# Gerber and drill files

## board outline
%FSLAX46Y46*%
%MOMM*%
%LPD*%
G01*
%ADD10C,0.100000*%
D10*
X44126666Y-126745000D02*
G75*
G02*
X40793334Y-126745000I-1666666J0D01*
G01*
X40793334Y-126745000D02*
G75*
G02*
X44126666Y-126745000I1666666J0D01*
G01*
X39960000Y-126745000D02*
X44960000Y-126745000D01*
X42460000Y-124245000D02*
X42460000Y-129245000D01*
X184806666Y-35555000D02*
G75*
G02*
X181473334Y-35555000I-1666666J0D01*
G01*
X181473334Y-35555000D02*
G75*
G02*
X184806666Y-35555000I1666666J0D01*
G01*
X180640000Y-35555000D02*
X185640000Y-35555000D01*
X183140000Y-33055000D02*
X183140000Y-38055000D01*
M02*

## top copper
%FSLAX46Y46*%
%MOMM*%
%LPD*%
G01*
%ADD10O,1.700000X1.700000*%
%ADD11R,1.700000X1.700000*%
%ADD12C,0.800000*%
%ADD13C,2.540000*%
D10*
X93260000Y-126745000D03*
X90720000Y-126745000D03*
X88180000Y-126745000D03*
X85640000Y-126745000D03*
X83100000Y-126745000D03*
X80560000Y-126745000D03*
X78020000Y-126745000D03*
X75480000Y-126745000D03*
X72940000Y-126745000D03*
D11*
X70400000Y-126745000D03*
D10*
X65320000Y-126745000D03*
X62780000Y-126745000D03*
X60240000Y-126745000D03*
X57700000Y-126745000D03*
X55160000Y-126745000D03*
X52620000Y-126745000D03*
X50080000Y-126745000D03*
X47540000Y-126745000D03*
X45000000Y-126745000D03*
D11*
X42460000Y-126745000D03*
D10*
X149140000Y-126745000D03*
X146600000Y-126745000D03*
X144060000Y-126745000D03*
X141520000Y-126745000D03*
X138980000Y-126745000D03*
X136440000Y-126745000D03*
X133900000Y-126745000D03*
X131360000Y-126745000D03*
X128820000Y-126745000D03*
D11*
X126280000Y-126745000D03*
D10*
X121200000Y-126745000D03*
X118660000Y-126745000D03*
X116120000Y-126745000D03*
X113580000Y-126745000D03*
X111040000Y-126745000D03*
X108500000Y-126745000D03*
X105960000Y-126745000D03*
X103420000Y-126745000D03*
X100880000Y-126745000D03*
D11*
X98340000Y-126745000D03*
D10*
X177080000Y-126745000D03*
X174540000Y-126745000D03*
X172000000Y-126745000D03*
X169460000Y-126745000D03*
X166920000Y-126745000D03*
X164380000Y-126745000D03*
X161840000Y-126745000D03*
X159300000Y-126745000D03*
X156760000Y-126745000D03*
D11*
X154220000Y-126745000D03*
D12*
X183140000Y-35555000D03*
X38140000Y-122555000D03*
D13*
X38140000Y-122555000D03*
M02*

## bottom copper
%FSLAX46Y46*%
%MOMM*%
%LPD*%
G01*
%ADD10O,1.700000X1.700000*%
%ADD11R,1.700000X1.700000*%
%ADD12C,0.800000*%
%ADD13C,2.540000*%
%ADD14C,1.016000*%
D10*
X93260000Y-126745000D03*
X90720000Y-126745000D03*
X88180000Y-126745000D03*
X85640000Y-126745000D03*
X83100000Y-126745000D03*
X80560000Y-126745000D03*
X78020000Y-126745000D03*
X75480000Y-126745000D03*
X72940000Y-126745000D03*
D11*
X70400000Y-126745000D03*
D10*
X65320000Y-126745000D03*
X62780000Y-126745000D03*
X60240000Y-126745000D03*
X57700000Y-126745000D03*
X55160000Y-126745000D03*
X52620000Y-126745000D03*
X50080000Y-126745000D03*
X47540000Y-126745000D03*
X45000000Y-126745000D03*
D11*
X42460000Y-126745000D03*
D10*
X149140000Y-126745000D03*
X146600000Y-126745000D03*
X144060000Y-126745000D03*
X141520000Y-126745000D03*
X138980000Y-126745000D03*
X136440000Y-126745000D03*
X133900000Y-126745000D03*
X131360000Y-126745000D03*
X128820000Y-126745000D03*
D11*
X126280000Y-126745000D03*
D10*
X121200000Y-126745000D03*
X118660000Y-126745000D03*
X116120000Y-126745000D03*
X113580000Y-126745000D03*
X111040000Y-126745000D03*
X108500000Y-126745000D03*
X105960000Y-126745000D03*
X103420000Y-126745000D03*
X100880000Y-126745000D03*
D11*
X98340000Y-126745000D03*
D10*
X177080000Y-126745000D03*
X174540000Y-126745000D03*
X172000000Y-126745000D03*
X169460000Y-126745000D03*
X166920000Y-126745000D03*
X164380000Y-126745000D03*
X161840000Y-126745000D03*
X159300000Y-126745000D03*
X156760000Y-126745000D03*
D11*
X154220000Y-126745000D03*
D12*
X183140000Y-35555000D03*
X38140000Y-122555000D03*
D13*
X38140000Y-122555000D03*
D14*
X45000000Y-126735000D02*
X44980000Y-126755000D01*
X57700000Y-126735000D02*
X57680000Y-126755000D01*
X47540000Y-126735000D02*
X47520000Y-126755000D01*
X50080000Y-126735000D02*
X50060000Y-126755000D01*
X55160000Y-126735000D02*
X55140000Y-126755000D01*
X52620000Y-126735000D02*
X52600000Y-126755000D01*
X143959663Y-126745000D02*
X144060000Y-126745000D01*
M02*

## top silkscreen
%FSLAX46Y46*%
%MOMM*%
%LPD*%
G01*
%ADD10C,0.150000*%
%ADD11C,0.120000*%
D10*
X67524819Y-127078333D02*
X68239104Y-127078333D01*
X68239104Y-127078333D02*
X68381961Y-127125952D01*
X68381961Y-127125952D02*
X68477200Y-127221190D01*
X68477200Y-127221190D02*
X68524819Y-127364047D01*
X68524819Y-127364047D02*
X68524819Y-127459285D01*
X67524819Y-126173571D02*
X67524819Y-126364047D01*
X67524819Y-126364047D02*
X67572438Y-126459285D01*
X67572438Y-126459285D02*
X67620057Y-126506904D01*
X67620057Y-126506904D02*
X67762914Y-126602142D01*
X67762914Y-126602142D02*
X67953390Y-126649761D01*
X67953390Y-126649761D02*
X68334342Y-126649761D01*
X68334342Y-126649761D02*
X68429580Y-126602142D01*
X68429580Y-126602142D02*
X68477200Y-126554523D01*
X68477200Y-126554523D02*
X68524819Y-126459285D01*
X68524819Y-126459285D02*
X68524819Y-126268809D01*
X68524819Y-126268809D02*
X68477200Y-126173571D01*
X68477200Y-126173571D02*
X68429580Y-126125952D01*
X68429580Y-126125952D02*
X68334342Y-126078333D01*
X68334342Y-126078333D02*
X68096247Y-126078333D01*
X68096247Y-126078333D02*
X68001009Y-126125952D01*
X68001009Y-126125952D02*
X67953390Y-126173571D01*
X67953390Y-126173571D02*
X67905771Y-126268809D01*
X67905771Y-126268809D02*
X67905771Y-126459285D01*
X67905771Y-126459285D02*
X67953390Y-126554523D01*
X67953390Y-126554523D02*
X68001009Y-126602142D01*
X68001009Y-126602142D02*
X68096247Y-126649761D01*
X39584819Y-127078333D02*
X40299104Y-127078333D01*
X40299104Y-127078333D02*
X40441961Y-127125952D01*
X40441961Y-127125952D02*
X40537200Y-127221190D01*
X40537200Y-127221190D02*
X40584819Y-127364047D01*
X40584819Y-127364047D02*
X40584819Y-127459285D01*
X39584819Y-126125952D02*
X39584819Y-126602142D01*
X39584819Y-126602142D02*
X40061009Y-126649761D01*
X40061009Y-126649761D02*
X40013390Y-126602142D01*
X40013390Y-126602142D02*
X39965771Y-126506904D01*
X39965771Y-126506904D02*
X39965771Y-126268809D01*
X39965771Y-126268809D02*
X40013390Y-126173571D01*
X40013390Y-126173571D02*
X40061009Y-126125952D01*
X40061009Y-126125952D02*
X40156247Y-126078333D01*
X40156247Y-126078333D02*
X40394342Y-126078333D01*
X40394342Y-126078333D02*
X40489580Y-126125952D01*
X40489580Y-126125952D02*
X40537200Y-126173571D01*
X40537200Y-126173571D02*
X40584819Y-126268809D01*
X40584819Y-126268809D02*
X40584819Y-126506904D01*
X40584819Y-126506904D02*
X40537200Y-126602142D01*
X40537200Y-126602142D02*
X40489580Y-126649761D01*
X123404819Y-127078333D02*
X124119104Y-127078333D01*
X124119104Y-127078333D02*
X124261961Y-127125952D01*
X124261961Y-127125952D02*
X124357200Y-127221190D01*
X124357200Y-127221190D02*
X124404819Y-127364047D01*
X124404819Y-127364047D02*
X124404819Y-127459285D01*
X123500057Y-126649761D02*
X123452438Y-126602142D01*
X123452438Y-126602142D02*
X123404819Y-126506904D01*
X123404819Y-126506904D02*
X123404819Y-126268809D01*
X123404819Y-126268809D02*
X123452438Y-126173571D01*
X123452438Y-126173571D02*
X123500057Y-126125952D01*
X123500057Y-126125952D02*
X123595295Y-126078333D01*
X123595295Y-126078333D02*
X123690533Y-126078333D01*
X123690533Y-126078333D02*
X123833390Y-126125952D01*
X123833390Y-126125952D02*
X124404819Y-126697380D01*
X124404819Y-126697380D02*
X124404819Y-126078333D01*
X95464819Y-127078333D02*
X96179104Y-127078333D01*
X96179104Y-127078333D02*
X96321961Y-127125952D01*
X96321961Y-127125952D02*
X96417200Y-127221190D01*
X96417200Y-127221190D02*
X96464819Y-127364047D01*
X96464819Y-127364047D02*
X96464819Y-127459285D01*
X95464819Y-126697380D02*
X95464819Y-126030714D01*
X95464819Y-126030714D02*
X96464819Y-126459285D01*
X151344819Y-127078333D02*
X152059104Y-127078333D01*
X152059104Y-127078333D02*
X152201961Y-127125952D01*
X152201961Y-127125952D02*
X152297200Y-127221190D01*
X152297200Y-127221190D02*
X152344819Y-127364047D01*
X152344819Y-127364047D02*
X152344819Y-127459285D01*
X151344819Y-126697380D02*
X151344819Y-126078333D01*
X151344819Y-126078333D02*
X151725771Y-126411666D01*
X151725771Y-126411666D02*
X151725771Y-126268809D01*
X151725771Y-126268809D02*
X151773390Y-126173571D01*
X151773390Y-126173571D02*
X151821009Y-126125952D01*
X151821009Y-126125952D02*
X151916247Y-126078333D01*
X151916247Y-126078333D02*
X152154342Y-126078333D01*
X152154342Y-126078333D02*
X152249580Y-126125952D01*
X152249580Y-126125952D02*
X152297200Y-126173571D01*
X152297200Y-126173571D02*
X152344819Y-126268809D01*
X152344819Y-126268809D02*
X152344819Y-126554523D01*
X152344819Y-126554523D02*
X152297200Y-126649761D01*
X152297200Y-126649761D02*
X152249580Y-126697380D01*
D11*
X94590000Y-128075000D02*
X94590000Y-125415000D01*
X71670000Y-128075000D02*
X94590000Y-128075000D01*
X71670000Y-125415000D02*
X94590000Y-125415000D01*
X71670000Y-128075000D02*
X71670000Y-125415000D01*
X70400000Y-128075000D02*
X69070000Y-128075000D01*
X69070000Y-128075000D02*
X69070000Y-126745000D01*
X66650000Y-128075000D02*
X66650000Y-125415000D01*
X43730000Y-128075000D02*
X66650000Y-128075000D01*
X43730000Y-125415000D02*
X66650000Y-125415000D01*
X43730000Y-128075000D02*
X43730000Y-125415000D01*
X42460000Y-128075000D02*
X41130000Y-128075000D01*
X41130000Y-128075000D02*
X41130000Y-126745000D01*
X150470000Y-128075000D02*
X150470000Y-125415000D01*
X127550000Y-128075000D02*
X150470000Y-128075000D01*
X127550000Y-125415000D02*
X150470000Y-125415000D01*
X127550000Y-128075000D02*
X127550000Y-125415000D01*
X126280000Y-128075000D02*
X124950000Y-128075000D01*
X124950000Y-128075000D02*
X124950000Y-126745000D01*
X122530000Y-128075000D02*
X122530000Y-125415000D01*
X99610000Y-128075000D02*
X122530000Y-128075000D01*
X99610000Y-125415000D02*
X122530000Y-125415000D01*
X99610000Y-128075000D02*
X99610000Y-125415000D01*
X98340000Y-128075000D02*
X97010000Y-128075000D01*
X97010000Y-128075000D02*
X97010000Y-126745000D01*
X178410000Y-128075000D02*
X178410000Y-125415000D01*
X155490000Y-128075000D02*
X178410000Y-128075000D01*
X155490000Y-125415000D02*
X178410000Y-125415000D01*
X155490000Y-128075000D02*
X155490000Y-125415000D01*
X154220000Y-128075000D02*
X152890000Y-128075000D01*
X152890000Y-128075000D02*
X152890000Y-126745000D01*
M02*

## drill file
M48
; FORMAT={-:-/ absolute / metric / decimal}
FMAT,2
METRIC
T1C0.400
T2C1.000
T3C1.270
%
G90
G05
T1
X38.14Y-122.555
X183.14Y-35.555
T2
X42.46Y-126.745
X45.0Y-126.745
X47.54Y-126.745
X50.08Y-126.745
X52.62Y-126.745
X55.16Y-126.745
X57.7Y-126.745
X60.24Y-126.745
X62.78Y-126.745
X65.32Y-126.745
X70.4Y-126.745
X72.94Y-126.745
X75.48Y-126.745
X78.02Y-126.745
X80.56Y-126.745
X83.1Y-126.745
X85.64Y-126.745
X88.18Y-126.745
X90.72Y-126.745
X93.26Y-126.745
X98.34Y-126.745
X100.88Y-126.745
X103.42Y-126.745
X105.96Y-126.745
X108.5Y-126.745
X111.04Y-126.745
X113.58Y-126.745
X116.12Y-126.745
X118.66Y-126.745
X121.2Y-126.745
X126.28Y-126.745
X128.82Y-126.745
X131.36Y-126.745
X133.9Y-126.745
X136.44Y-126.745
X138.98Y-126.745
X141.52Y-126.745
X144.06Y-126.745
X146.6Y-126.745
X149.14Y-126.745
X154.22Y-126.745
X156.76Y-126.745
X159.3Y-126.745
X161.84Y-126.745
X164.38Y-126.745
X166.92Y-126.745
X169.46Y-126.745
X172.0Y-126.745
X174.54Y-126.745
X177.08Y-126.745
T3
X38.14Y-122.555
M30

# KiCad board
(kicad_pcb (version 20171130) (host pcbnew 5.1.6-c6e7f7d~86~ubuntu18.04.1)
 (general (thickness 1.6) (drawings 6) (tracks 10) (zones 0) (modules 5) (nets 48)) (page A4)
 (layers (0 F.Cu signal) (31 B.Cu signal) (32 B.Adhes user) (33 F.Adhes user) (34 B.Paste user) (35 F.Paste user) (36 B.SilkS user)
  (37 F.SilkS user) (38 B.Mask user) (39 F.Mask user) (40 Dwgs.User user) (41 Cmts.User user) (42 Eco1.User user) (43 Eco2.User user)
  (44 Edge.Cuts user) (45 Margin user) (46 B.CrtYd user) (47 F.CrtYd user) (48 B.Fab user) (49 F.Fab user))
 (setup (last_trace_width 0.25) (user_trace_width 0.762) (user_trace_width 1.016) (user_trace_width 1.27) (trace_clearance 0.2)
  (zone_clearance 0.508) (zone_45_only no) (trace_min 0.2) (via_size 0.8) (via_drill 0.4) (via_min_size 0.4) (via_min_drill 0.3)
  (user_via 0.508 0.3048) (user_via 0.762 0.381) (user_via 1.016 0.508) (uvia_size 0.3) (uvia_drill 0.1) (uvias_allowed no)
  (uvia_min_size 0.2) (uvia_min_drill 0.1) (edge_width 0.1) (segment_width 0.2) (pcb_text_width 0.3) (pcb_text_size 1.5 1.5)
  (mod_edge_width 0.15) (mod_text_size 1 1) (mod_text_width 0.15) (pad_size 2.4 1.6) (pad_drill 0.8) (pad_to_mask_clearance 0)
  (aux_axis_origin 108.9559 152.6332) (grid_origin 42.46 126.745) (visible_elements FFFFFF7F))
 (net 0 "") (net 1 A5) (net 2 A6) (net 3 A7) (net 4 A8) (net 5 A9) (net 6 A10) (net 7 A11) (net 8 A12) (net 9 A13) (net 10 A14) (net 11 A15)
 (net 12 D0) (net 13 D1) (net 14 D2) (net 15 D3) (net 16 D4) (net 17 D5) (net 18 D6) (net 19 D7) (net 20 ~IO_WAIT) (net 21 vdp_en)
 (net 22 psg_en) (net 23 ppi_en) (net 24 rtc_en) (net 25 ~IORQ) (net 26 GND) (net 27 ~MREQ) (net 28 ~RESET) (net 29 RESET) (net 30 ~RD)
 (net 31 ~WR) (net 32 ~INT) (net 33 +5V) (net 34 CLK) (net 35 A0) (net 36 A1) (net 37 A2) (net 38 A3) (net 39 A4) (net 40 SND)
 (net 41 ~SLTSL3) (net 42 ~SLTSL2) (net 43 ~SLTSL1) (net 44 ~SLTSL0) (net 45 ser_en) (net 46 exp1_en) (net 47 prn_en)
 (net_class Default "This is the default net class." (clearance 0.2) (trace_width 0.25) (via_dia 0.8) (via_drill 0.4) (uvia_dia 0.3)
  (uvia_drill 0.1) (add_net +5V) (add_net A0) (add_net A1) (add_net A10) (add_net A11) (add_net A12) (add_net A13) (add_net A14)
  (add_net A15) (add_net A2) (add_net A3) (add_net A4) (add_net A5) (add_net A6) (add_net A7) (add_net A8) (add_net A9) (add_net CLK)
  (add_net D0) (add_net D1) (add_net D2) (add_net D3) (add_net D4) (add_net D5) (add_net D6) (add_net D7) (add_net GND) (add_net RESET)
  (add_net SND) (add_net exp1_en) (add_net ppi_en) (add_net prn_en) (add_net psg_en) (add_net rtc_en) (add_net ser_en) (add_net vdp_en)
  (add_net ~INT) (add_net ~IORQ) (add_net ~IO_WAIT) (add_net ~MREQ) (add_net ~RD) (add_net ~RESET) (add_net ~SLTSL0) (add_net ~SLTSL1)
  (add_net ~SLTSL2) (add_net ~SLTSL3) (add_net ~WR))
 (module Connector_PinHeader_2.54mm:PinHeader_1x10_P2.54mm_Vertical (layer F.Cu) (at 70.4 126.745 90)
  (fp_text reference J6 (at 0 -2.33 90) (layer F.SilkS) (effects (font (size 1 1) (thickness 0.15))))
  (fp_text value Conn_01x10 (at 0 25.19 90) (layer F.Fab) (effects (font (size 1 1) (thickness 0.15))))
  (fp_line (start -1.33 24.19) (end 1.33 24.19) (layer F.SilkS) (width 0.12))
  (fp_line (start -1.33 1.27) (end -1.33 24.19) (layer F.SilkS) (width 0.12))
  (fp_line (start 1.33 1.27) (end 1.33 24.19) (layer F.SilkS) (width 0.12))
  (fp_line (start -1.33 1.27) (end 1.33 1.27) (layer F.SilkS) (width 0.12))
  (fp_line (start -1.33 0) (end -1.33 -1.33) (layer F.SilkS) (width 0.12))
  (fp_line (start -1.33 -1.33) (end 0 -1.33) (layer F.SilkS) (width 0.12))
  (pad 10 thru_hole oval (at 0 22.86 90) (size 1.7 1.7) (drill 1) (layers *.Cu *.Mask) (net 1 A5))
  (pad 9 thru_hole oval (at 0 20.32 90) (size 1.7 1.7) (drill 1) (layers *.Cu *.Mask) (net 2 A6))
  (pad 8 thru_hole oval (at 0 17.78 90) (size 1.7 1.7) (drill 1) (layers *.Cu *.Mask) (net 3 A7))
  (pad 7 thru_hole oval (at 0 15.24 90) (size 1.7 1.7) (drill 1) (layers *.Cu *.Mask) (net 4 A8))
  (pad 6 thru_hole oval (at 0 12.7 90) (size 1.7 1.7) (drill 1) (layers *.Cu *.Mask) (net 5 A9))
  (pad 5 thru_hole oval (at 0 10.16 90) (size 1.7 1.7) (drill 1) (layers *.Cu *.Mask) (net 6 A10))
  (pad 4 thru_hole oval (at 0 7.62 90) (size 1.7 1.7) (drill 1) (layers *.Cu *.Mask) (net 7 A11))
  (pad 3 thru_hole oval (at 0 5.08 90) (size 1.7 1.7) (drill 1) (layers *.Cu *.Mask) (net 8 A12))
  (pad 2 thru_hole oval (at 0 2.54 90) (size 1.7 1.7) (drill 1) (layers *.Cu *.Mask) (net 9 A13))
  (pad 1 thru_hole rect (at 0 0 90) (size 1.7 1.7) (drill 1) (layers *.Cu *.Mask) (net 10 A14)))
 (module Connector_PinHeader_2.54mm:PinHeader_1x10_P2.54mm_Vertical (layer F.Cu) (at 42.46 126.745 90)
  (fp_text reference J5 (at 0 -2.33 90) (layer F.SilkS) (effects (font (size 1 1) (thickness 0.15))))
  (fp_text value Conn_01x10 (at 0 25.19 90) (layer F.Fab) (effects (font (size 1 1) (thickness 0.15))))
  (fp_line (start -1.33 24.19) (end 1.33 24.19) (layer F.SilkS) (width 0.12))
  (fp_line (start -1.33 1.27) (end -1.33 24.19) (layer F.SilkS) (width 0.12))
  (fp_line (start 1.33 1.27) (end 1.33 24.19) (layer F.SilkS) (width 0.12))
  (fp_line (start -1.33 1.27) (end 1.33 1.27) (layer F.SilkS) (width 0.12))
  (fp_line (start -1.33 0) (end -1.33 -1.33) (layer F.SilkS) (width 0.12))
  (fp_line (start -1.33 -1.33) (end 0 -1.33) (layer F.SilkS) (width 0.12))
  (pad 10 thru_hole oval (at 0 22.86 90) (size 1.7 1.7) (drill 1) (layers *.Cu *.Mask) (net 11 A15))
  (pad 9 thru_hole oval (at 0 20.32 90) (size 1.7 1.7) (drill 1) (layers *.Cu *.Mask) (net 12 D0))
  (pad 8 thru_hole oval (at 0 17.78 90) (size 1.7 1.7) (drill 1) (layers *.Cu *.Mask) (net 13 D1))
  (pad 7 thru_hole oval (at 0 15.24 90) (size 1.7 1.7) (drill 1) (layers *.Cu *.Mask) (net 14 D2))
  (pad 6 thru_hole oval (at 0 12.7 90) (size 1.7 1.7) (drill 1) (layers *.Cu *.Mask) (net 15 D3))
  (pad 5 thru_hole oval (at 0 10.16 90) (size 1.7 1.7) (drill 1) (layers *.Cu *.Mask) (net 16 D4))
  (pad 4 thru_hole oval (at 0 7.62 90) (size 1.7 1.7) (drill 1) (layers *.Cu *.Mask) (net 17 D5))
  (pad 3 thru_hole oval (at 0 5.08 90) (size 1.7 1.7) (drill 1) (layers *.Cu *.Mask) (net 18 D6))
  (pad 2 thru_hole oval (at 0 2.54 90) (size 1.7 1.7) (drill 1) (layers *.Cu *.Mask) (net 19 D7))
  (pad 1 thru_hole rect (at 0 0 90) (size 1.7 1.7) (drill 1) (layers *.Cu *.Mask) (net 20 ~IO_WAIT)))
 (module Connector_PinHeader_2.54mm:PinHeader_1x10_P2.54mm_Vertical (layer F.Cu) (at 126.28 126.745 90)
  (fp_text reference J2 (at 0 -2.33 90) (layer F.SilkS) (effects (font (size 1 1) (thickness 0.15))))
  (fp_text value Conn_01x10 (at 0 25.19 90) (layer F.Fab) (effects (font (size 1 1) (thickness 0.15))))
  (fp_line (start -1.33 24.19) (end 1.33 24.19) (layer F.SilkS) (width 0.12))
  (fp_line (start -1.33 1.27) (end -1.33 24.19) (layer F.SilkS) (width 0.12))
  (fp_line (start 1.33 1.27) (end 1.33 24.19) (layer F.SilkS) (width 0.12))
  (fp_line (start -1.33 1.27) (end 1.33 1.27) (layer F.SilkS) (width 0.12))
  (fp_line (start -1.33 0) (end -1.33 -1.33) (layer F.SilkS) (width 0.12))
  (fp_line (start -1.33 -1.33) (end 0 -1.33) (layer F.SilkS) (width 0.12))
  (pad 10 thru_hole oval (at 0 22.86 90) (size 1.7 1.7) (drill 1) (layers *.Cu *.Mask) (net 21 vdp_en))
  (pad 9 thru_hole oval (at 0 20.32 90) (size 1.7 1.7) (drill 1) (layers *.Cu *.Mask) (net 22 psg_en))
  (pad 8 thru_hole oval (at 0 17.78 90) (size 1.7 1.7) (drill 1) (layers *.Cu *.Mask) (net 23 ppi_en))
  (pad 7 thru_hole oval (at 0 15.24 90) (size 1.7 1.7) (drill 1) (layers *.Cu *.Mask) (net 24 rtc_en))
  (pad 6 thru_hole oval (at 0 12.7 90) (size 1.7 1.7) (drill 1) (layers *.Cu *.Mask) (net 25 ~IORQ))
  (pad 5 thru_hole oval (at 0 10.16 90) (size 1.7 1.7) (drill 1) (layers *.Cu *.Mask) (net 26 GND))
  (pad 4 thru_hole oval (at 0 7.62 90) (size 1.7 1.7) (drill 1) (layers *.Cu *.Mask) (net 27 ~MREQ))
  (pad 3 thru_hole oval (at 0 5.08 90) (size 1.7 1.7) (drill 1) (layers *.Cu *.Mask) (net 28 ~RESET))
  (pad 2 thru_hole oval (at 0 2.54 90) (size 1.7 1.7) (drill 1) (layers *.Cu *.Mask) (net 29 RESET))
  (pad 1 thru_hole rect (at 0 0 90) (size 1.7 1.7) (drill 1) (layers *.Cu *.Mask) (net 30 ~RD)))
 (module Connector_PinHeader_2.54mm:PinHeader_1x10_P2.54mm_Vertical (layer F.Cu) (at 98.34 126.745 90)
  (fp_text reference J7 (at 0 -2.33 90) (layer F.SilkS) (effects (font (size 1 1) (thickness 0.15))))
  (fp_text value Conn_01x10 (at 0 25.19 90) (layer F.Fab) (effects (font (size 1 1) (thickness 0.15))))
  (fp_line (start -1.33 24.19) (end 1.33 24.19) (layer F.SilkS) (width 0.12))
  (fp_line (start -1.33 1.27) (end -1.33 24.19) (layer F.SilkS) (width 0.12))
  (fp_line (start 1.33 1.27) (end 1.33 24.19) (layer F.SilkS) (width 0.12))
  (fp_line (start -1.33 1.27) (end 1.33 1.27) (layer F.SilkS) (width 0.12))
  (fp_line (start -1.33 0) (end -1.33 -1.33) (layer F.SilkS) (width 0.12))
  (fp_line (start -1.33 -1.33) (end 0 -1.33) (layer F.SilkS) (width 0.12))
  (pad 10 thru_hole oval (at 0 22.86 90) (size 1.7 1.7) (drill 1) (layers *.Cu *.Mask) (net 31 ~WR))
  (pad 9 thru_hole oval (at 0 20.32 90) (size 1.7 1.7) (drill 1) (layers *.Cu *.Mask) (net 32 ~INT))
  (pad 8 thru_hole oval (at 0 17.78 90) (size 1.7 1.7) (drill 1) (layers *.Cu *.Mask) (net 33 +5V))
  (pad 7 thru_hole oval (at 0 15.24 90) (size 1.7 1.7) (drill 1) (layers *.Cu *.Mask) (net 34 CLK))
  (pad 6 thru_hole oval (at 0 12.7 90) (size 1.7 1.7) (drill 1) (layers *.Cu *.Mask) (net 26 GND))
  (pad 5 thru_hole oval (at 0 10.16 90) (size 1.7 1.7) (drill 1) (layers *.Cu *.Mask) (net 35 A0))
  (pad 4 thru_hole oval (at 0 7.62 90) (size 1.7 1.7) (drill 1) (layers *.Cu *.Mask) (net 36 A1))
  (pad 3 thru_hole oval (at 0 5.08 90) (size 1.7 1.7) (drill 1) (layers *.Cu *.Mask) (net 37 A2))
  (pad 2 thru_hole oval (at 0 2.54 90) (size 1.7 1.7) (drill 1) (layers *.Cu *.Mask) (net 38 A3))
  (pad 1 thru_hole rect (at 0 0 90) (size 1.7 1.7) (drill 1) (layers *.Cu *.Mask) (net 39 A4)))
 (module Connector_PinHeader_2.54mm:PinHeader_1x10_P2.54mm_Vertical (layer F.Cu) (at 154.22 126.745 90)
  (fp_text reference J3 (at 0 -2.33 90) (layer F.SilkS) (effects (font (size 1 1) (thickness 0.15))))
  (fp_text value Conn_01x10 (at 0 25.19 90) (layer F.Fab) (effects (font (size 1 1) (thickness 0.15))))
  (fp_line (start -1.33 24.19) (end 1.33 24.19) (layer F.SilkS) (width 0.12))
  (fp_line (start -1.33 1.27) (end -1.33 24.19) (layer F.SilkS) (width 0.12))
  (fp_line (start 1.33 1.27) (end 1.33 24.19) (layer F.SilkS) (width 0.12))
  (fp_line (start -1.33 1.27) (end 1.33 1.27) (layer F.SilkS) (width 0.12))
  (fp_line (start -1.33 0) (end -1.33 -1.33) (layer F.SilkS) (width 0.12))
  (fp_line (start -1.33 -1.33) (end 0 -1.33) (layer F.SilkS) (width 0.12))
  (pad 10 thru_hole oval (at 0 22.86 90) (size 1.7 1.7) (drill 1) (layers *.Cu *.Mask) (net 26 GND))
  (pad 9 thru_hole oval (at 0 20.32 90) (size 1.7 1.7) (drill 1) (layers *.Cu *.Mask) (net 33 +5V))
  (pad 8 thru_hole oval (at 0 17.78 90) (size 1.7 1.7) (drill 1) (layers *.Cu *.Mask) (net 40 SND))
  (pad 7 thru_hole oval (at 0 15.24 90) (size 1.7 1.7) (drill 1) (layers *.Cu *.Mask) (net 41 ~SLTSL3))
  (pad 6 thru_hole oval (at 0 12.7 90) (size 1.7 1.7) (drill 1) (layers *.Cu *.Mask) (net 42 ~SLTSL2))
  (pad 5 thru_hole oval (at 0 10.16 90) (size 1.7 1.7) (drill 1) (layers *.Cu *.Mask) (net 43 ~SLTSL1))
  (pad 4 thru_hole oval (at 0 7.62 90) (size 1.7 1.7) (drill 1) (layers *.Cu *.Mask) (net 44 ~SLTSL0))
  (pad 3 thru_hole oval (at 0 5.08 90) (size 1.7 1.7) (drill 1) (layers *.Cu *.Mask) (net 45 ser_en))
  (pad 2 thru_hole oval (at 0 2.54 90) (size 1.7 1.7) (drill 1) (layers *.Cu *.Mask) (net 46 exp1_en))
  (pad 1 thru_hole rect (at 0 0 90) (size 1.7 1.7) (drill 1) (layers *.Cu *.Mask) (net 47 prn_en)))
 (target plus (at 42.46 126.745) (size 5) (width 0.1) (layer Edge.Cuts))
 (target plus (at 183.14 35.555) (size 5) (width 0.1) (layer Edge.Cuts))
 (via (at 183.14 35.555) (size 0.8) (drill 0.4) (layers F.Cu B.Cu) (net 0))
 (via (at 38.14 122.555) (size 0.8) (drill 0.4) (layers F.Cu B.Cu) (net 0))
 (via (at 38.14 122.555) (size 2.54) (drill 1.27) (layers F.Cu B.Cu) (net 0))
 (segment (start 45 126.735) (end 44.98 126.755) (width 1.016) (layer B.Cu) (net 19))
 (segment (start 57.7 126.735) (end 57.68 126.755) (width 1.016) (layer B.Cu) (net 14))
 (segment (start 47.54 126.735) (end 47.52 126.755) (width 1.016) (layer B.Cu) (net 18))
 (segment (start 50.08 126.735) (end 50.06 126.755) (width 1.016) (layer B.Cu) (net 17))
 (segment (start 55.16 126.735) (end 55.14 126.755) (width 1.016) (layer B.Cu) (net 15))
 (segment (start 52.62 126.735) (end 52.6 126.755) (width 1.016) (layer B.Cu) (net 16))
 (segment (start 143.959663 126.745) (end 144.06 126.745) (width 1.016) (layer B.Cu) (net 23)))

